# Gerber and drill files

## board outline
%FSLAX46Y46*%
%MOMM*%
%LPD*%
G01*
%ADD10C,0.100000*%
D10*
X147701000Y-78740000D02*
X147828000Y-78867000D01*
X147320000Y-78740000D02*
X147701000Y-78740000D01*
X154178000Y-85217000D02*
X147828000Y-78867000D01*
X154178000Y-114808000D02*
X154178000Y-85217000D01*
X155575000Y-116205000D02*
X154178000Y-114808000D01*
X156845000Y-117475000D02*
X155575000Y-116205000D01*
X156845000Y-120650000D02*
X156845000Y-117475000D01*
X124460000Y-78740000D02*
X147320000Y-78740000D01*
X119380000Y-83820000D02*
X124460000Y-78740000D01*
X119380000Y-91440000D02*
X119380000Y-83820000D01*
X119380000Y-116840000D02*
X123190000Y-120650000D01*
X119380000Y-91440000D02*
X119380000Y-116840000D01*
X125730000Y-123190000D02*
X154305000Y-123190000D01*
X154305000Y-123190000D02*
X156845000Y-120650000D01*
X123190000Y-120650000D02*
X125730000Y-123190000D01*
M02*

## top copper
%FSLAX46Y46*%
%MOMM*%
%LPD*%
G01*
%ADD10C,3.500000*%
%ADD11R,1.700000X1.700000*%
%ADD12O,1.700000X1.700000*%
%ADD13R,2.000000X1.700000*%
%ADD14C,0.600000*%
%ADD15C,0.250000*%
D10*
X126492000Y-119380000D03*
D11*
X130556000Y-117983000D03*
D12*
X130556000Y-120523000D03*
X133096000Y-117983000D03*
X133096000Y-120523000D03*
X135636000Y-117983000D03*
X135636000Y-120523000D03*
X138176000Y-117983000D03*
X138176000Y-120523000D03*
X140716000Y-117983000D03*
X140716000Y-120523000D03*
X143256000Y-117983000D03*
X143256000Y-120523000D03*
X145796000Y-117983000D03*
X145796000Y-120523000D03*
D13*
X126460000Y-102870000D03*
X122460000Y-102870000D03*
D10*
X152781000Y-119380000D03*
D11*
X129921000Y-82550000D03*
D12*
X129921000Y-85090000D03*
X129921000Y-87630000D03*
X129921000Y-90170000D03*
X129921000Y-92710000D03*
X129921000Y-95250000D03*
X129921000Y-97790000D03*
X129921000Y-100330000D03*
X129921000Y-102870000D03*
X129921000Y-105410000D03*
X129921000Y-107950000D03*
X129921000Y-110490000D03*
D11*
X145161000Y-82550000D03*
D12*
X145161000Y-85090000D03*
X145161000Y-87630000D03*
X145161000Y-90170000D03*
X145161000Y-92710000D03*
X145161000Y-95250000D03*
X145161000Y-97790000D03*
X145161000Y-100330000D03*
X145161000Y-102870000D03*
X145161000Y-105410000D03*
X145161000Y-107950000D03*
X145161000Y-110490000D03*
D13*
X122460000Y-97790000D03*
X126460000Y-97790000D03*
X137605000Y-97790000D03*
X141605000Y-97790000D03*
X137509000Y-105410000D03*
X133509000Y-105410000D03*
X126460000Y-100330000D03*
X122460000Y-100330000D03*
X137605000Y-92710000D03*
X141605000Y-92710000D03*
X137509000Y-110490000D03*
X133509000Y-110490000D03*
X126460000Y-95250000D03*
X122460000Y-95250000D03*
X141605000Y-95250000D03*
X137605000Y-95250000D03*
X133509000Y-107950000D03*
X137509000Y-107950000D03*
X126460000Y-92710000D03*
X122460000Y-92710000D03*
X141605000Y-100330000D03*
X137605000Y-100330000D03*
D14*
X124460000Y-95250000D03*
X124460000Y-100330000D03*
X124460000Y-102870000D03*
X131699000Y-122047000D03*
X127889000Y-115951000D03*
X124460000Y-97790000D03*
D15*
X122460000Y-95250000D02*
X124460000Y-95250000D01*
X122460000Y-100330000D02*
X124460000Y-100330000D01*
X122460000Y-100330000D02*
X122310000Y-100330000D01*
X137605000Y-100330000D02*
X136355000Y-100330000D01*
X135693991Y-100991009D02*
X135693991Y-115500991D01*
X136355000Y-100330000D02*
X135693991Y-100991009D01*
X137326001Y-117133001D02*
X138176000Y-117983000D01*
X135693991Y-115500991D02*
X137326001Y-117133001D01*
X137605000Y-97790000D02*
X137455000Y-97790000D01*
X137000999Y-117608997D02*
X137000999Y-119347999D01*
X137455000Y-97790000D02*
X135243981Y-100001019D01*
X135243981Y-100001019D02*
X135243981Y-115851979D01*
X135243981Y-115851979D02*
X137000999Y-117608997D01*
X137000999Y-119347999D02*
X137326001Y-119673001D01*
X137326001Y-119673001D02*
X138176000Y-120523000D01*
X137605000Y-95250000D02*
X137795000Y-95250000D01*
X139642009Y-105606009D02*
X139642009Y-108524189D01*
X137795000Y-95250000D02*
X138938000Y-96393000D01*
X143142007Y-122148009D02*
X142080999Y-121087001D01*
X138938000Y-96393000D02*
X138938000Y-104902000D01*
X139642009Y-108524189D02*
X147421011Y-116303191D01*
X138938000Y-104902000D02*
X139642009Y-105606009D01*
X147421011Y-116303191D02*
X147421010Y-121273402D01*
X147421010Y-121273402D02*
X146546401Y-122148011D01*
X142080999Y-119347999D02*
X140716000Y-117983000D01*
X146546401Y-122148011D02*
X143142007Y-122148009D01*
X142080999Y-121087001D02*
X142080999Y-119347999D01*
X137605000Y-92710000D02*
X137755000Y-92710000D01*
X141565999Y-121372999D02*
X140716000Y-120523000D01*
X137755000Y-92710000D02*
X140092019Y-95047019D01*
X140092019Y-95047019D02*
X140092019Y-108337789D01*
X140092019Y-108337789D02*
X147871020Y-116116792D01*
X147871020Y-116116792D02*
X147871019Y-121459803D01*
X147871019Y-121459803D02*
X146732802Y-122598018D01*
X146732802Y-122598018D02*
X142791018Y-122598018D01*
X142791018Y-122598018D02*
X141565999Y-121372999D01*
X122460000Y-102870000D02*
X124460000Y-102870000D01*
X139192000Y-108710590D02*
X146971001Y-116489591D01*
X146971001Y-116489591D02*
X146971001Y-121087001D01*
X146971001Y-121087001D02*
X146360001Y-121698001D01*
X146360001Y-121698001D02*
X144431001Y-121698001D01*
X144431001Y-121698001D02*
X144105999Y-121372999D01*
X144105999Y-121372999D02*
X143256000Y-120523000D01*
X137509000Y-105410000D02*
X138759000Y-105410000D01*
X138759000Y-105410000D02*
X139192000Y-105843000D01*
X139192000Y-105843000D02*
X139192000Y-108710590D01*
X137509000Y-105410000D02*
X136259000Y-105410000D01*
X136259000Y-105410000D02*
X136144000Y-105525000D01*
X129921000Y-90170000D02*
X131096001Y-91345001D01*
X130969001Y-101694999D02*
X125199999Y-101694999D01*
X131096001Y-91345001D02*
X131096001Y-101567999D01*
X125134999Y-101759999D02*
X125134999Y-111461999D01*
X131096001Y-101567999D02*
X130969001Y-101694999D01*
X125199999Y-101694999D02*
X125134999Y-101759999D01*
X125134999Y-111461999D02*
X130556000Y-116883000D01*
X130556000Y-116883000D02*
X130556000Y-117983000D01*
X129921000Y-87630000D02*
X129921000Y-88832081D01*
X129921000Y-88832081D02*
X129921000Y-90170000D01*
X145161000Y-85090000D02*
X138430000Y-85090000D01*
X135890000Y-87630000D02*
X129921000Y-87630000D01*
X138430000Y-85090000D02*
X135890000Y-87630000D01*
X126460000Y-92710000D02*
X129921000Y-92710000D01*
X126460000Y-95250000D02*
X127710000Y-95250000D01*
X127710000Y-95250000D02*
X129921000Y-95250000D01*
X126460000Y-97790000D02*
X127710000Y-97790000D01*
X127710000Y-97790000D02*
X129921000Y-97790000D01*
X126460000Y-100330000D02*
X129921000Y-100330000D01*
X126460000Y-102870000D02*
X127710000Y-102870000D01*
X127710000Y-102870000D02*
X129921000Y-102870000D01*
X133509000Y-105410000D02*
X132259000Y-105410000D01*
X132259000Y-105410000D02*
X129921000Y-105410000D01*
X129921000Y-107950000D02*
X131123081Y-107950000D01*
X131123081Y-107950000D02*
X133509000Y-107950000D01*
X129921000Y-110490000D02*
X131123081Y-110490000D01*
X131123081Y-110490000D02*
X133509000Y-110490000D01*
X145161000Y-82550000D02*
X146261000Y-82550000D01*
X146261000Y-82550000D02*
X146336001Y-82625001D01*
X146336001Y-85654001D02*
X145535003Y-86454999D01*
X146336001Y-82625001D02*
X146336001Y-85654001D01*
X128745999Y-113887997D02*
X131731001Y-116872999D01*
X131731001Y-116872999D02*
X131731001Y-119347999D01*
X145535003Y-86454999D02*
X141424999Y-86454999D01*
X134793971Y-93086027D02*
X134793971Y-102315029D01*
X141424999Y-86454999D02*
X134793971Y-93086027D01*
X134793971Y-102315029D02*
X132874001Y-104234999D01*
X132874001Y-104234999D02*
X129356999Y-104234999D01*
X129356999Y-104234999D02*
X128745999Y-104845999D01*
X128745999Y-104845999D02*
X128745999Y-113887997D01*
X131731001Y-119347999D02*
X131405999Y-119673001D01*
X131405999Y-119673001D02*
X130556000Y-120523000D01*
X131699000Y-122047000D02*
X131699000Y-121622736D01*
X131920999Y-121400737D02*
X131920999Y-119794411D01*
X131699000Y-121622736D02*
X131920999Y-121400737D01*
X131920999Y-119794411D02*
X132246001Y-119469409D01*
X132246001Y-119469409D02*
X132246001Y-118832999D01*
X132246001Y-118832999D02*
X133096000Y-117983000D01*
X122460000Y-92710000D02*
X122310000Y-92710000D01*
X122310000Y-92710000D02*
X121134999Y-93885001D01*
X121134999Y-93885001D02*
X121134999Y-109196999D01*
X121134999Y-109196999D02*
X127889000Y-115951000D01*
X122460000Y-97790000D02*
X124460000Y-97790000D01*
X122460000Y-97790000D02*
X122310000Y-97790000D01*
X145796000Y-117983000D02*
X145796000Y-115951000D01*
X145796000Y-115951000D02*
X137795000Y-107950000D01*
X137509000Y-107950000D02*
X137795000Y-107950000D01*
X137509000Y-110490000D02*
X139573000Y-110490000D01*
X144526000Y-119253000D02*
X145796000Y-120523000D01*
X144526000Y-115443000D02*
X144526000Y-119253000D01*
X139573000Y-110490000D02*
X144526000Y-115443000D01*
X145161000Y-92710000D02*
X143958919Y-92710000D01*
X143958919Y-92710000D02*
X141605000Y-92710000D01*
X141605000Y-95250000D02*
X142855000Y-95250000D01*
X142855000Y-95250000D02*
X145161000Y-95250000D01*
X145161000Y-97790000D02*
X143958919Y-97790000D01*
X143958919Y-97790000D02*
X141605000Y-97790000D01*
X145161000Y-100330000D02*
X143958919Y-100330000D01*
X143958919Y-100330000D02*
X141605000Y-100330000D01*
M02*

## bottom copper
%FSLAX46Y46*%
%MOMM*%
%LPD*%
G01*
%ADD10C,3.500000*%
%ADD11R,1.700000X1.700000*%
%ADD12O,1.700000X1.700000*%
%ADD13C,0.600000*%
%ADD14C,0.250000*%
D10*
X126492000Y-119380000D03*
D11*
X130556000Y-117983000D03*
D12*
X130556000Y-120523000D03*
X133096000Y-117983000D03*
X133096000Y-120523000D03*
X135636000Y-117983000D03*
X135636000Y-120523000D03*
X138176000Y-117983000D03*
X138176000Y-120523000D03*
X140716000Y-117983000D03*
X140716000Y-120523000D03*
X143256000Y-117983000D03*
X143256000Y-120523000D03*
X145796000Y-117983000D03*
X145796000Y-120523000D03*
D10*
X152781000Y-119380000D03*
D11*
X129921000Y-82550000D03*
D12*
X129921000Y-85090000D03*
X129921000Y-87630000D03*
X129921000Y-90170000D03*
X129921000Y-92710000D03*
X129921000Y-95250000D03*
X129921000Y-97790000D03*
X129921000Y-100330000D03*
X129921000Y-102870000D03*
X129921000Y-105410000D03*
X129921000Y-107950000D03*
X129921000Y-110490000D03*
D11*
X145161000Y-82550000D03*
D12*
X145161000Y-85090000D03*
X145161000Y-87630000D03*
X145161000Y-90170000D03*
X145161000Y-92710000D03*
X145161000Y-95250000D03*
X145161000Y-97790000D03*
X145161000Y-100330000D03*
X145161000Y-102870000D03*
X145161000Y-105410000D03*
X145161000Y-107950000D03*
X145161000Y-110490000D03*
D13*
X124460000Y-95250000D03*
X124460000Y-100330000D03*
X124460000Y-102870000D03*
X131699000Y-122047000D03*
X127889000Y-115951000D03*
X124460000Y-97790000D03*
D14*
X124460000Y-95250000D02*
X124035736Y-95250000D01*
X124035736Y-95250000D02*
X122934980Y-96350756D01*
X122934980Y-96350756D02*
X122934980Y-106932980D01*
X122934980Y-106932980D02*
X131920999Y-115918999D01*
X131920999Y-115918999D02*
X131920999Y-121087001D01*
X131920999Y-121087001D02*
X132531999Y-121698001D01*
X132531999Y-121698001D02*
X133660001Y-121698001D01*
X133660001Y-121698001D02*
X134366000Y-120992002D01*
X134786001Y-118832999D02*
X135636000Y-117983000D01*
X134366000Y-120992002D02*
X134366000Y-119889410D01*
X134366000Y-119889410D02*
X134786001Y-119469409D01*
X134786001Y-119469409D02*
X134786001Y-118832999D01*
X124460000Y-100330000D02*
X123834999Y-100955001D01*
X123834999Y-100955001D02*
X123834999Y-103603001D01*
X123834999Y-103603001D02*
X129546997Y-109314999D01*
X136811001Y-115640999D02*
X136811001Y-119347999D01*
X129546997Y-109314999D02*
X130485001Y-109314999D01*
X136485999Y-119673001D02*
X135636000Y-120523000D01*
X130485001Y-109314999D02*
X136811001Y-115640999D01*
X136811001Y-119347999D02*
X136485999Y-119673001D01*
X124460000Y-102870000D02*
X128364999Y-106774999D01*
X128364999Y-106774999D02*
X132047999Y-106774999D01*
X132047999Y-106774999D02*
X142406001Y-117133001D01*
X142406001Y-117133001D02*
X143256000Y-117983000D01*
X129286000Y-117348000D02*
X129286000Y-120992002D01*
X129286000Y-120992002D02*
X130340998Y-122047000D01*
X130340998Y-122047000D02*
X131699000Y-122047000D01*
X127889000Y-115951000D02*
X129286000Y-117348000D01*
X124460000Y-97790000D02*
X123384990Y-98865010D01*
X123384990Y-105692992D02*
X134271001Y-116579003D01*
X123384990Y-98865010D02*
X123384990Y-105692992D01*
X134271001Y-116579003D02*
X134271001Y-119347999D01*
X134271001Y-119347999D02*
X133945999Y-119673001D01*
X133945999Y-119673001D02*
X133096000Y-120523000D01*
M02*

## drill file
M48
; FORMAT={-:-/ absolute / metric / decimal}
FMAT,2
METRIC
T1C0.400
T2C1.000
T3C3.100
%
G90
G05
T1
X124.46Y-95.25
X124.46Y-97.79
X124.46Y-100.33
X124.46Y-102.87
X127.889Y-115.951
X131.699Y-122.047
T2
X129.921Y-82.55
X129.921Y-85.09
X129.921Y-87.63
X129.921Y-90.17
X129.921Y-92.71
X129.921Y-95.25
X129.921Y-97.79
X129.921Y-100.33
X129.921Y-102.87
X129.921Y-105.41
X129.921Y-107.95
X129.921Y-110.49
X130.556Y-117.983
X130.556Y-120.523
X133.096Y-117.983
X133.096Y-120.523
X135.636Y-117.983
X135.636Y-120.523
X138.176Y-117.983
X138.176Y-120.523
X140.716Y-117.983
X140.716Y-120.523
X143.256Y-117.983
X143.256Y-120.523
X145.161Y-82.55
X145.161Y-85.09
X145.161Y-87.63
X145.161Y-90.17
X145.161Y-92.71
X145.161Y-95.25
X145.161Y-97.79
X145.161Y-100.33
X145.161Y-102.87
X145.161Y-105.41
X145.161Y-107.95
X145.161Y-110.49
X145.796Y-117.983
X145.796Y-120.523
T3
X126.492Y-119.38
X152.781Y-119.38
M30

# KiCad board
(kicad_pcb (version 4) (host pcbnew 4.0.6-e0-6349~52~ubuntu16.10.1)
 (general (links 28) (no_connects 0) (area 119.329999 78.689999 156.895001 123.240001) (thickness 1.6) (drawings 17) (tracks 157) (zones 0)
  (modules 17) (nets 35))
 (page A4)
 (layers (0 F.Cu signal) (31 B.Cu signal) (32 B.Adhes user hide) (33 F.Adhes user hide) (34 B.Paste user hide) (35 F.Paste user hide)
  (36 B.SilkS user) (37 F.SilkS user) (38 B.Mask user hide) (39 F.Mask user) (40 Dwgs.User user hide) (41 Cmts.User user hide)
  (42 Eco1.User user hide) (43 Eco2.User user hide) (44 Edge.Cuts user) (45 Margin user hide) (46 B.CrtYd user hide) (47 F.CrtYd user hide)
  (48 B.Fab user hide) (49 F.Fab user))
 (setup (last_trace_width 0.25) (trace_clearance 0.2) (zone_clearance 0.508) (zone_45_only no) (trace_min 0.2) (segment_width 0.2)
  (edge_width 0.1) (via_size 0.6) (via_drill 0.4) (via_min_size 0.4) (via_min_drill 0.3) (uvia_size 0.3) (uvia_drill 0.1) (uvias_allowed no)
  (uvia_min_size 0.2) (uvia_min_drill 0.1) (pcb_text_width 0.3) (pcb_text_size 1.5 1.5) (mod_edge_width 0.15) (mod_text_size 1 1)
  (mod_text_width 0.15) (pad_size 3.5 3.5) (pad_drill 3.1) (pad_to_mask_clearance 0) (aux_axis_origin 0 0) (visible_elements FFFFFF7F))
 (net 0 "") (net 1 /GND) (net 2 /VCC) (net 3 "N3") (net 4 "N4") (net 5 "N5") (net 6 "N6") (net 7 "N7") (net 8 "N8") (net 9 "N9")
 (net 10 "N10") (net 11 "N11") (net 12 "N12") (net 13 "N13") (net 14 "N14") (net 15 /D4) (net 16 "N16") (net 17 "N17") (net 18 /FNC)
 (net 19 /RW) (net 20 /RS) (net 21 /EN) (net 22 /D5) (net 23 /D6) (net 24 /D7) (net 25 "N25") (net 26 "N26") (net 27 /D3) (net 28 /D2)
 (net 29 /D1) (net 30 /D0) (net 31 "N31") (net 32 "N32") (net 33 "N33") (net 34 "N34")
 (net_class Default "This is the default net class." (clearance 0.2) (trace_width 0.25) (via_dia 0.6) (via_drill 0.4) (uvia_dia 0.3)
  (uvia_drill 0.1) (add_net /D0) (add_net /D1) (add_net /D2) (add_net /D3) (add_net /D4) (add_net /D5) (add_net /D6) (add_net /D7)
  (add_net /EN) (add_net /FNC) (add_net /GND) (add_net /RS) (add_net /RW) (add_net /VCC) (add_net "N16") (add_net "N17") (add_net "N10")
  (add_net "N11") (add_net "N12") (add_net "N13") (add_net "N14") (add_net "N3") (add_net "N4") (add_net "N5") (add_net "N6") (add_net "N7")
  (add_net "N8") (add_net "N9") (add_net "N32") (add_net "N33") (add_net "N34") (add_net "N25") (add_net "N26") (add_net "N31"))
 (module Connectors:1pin (layer F.Cu) (at 126.492 119.38)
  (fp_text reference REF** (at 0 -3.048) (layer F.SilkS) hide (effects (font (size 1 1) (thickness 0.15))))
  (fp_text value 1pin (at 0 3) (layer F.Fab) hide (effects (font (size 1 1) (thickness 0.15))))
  (pad 1 thru_hole circle (at 0 0) (size 3.5 3.5) (drill 3.1) (layers *.Cu *.Mask)))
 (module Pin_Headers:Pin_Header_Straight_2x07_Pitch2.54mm (layer B.Cu) (at 130.556 117.983 270)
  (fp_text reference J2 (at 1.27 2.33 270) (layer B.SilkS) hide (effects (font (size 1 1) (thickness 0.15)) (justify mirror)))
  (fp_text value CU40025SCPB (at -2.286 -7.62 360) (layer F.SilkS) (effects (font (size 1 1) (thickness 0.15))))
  (pad 1 thru_hole rect (at 0 0 270) (size 1.7 1.7) (drill 1) (layers *.Cu *.Mask) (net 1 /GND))
  (pad 2 thru_hole oval (at 2.54 0 270) (size 1.7 1.7) (drill 1) (layers *.Cu *.Mask) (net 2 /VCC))
  (pad 3 thru_hole oval (at 0 -2.54 270) (size 1.7 1.7) (drill 1) (layers *.Cu *.Mask) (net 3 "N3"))
  (pad 4 thru_hole oval (at 2.54 -2.54 270) (size 1.7 1.7) (drill 1) (layers *.Cu *.Mask) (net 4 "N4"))
  (pad 5 thru_hole oval (at 0 -5.08 270) (size 1.7 1.7) (drill 1) (layers *.Cu *.Mask) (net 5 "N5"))
  (pad 6 thru_hole oval (at 2.54 -5.08 270) (size 1.7 1.7) (drill 1) (layers *.Cu *.Mask) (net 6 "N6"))
  (pad 7 thru_hole oval (at 0 -7.62 270) (size 1.7 1.7) (drill 1) (layers *.Cu *.Mask) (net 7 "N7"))
  (pad 8 thru_hole oval (at 2.54 -7.62 270) (size 1.7 1.7) (drill 1) (layers *.Cu *.Mask) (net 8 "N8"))
  (pad 9 thru_hole oval (at 0 -10.16 270) (size 1.7 1.7) (drill 1) (layers *.Cu *.Mask) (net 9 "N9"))
  (pad 10 thru_hole oval (at 2.54 -10.16 270) (size 1.7 1.7) (drill 1) (layers *.Cu *.Mask) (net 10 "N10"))
  (pad 11 thru_hole oval (at 0 -12.7 270) (size 1.7 1.7) (drill 1) (layers *.Cu *.Mask) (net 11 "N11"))
  (pad 12 thru_hole oval (at 2.54 -12.7 270) (size 1.7 1.7) (drill 1) (layers *.Cu *.Mask) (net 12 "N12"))
  (pad 13 thru_hole oval (at 0 -15.24 270) (size 1.7 1.7) (drill 1) (layers *.Cu *.Mask) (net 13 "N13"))
  (pad 14 thru_hole oval (at 2.54 -15.24 270) (size 1.7 1.7) (drill 1) (layers *.Cu *.Mask) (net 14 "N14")))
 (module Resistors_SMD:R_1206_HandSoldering (layer F.Cu) (at 124.46 102.87 180)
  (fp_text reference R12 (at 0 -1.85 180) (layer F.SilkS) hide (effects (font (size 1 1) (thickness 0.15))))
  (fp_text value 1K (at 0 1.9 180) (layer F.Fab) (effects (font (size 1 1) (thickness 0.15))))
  (pad 1 smd rect (at -2 0 180) (size 2 1.7) (layers F.Cu F.Paste F.Mask) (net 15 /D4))
  (pad 2 smd rect (at 2 0 180) (size 2 1.7) (layers F.Cu F.Paste F.Mask) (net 11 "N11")))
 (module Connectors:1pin (layer F.Cu) (at 152.781 119.38)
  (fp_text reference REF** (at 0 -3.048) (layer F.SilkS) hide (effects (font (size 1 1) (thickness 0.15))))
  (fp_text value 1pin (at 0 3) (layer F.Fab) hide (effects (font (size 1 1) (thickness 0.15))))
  (pad 1 thru_hole circle (at 0 0) (size 3.5 3.5) (drill 3.1) (layers *.Cu *.Mask)))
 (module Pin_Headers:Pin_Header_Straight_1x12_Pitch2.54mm (layer F.Cu) (at 129.921 82.55)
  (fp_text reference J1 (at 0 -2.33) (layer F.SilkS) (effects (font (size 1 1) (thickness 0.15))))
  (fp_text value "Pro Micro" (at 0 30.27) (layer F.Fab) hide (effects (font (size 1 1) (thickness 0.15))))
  (pad 1 thru_hole rect (at 0 0) (size 1.7 1.7) (drill 1) (layers *.Cu *.Mask) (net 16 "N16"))
  (pad 2 thru_hole oval (at 0 2.54) (size 1.7 1.7) (drill 1) (layers *.Cu *.Mask) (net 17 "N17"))
  (pad 3 thru_hole oval (at 0 5.08) (size 1.7 1.7) (drill 1) (layers *.Cu *.Mask) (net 1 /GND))
  (pad 4 thru_hole oval (at 0 7.62) (size 1.7 1.7) (drill 1) (layers *.Cu *.Mask) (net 1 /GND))
  (pad 5 thru_hole oval (at 0 10.16) (size 1.7 1.7) (drill 1) (layers *.Cu *.Mask) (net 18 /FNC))
  (pad 6 thru_hole oval (at 0 12.7) (size 1.7 1.7) (drill 1) (layers *.Cu *.Mask) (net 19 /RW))
  (pad 7 thru_hole oval (at 0 15.24) (size 1.7 1.7) (drill 1) (layers *.Cu *.Mask) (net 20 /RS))
  (pad 8 thru_hole oval (at 0 17.78) (size 1.7 1.7) (drill 1) (layers *.Cu *.Mask) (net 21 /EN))
  (pad 9 thru_hole oval (at 0 20.32) (size 1.7 1.7) (drill 1) (layers *.Cu *.Mask) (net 15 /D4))
  (pad 10 thru_hole oval (at 0 22.86) (size 1.7 1.7) (drill 1) (layers *.Cu *.Mask) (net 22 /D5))
  (pad 11 thru_hole oval (at 0 25.4) (size 1.7 1.7) (drill 1) (layers *.Cu *.Mask) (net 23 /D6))
  (pad 12 thru_hole oval (at 0 27.94) (size 1.7 1.7) (drill 1) (layers *.Cu *.Mask) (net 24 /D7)))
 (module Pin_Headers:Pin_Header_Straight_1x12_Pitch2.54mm (layer F.Cu) (at 145.161 82.55)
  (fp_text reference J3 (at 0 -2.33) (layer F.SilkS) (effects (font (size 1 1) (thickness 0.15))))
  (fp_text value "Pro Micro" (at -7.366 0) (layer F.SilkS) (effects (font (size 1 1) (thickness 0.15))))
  (pad 1 thru_hole rect (at 0 0) (size 1.7 1.7) (drill 1) (layers *.Cu *.Mask) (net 2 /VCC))
  (pad 2 thru_hole oval (at 0 2.54) (size 1.7 1.7) (drill 1) (layers *.Cu *.Mask) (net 1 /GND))
  (pad 3 thru_hole oval (at 0 5.08) (size 1.7 1.7) (drill 1) (layers *.Cu *.Mask) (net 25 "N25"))
  (pad 4 thru_hole oval (at 0 7.62) (size 1.7 1.7) (drill 1) (layers *.Cu *.Mask) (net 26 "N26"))
  (pad 5 thru_hole oval (at 0 10.16) (size 1.7 1.7) (drill 1) (layers *.Cu *.Mask) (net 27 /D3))
  (pad 6 thru_hole oval (at 0 12.7) (size 1.7 1.7) (drill 1) (layers *.Cu *.Mask) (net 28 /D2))
  (pad 7 thru_hole oval (at 0 15.24) (size 1.7 1.7) (drill 1) (layers *.Cu *.Mask) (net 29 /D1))
  (pad 8 thru_hole oval (at 0 17.78) (size 1.7 1.7) (drill 1) (layers *.Cu *.Mask) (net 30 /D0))
  (pad 9 thru_hole oval (at 0 20.32) (size 1.7 1.7) (drill 1) (layers *.Cu *.Mask) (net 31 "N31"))
  (pad 10 thru_hole oval (at 0 22.86) (size 1.7 1.7) (drill 1) (layers *.Cu *.Mask) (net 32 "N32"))
  (pad 11 thru_hole oval (at 0 25.4) (size 1.7 1.7) (drill 1) (layers *.Cu *.Mask) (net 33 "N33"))
  (pad 12 thru_hole oval (at 0 27.94) (size 1.7 1.7) (drill 1) (layers *.Cu *.Mask) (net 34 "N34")))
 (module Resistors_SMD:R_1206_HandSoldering (layer F.Cu) (at 124.46 97.79)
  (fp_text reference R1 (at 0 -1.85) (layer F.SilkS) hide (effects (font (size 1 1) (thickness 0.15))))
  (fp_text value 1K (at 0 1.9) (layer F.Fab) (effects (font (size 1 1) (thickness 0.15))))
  (pad 1 smd rect (at -2 0) (size 2 1.7) (layers F.Cu F.Paste F.Mask) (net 4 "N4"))
  (pad 2 smd rect (at 2 0) (size 2 1.7) (layers F.Cu F.Paste F.Mask) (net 20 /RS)))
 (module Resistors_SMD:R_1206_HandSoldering (layer F.Cu) (at 139.605 97.79)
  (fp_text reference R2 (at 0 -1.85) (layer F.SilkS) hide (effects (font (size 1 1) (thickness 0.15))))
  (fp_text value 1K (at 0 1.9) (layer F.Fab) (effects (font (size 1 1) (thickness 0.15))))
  (pad 1 smd rect (at -2 0) (size 2 1.7) (layers F.Cu F.Paste F.Mask) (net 8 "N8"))
  (pad 2 smd rect (at 2 0) (size 2 1.7) (layers F.Cu F.Paste F.Mask) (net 29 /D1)))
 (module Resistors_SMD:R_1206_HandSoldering (layer F.Cu) (at 135.509 105.41 180)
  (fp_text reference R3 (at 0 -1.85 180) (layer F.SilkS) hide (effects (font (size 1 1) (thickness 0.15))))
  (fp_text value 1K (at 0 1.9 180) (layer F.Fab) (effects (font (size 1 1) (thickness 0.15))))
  (pad 1 smd rect (at -2 0 180) (size 2 1.7) (layers F.Cu F.Paste F.Mask) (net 12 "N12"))
  (pad 2 smd rect (at 2 0 180) (size 2 1.7) (layers F.Cu F.Paste F.Mask) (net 22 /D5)))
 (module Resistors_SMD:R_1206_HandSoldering (layer F.Cu) (at 124.46 100.33 180)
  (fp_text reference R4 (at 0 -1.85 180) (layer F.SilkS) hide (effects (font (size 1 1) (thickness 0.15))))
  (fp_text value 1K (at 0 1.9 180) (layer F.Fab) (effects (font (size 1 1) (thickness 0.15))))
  (pad 1 smd rect (at -2 0 180) (size 2 1.7) (layers F.Cu F.Paste F.Mask) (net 21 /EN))
  (pad 2 smd rect (at 2 0 180) (size 2 1.7) (layers F.Cu F.Paste F.Mask) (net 6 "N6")))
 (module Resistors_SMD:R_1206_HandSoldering (layer F.Cu) (at 139.605 92.71)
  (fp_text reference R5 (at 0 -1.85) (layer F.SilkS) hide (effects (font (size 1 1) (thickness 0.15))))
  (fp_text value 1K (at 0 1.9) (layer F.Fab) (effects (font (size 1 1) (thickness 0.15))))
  (pad 1 smd rect (at -2 0) (size 2 1.7) (layers F.Cu F.Paste F.Mask) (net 10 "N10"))
  (pad 2 smd rect (at 2 0) (size 2 1.7) (layers F.Cu F.Paste F.Mask) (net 27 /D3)))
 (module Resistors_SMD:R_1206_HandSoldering (layer F.Cu) (at 135.509 110.49 180)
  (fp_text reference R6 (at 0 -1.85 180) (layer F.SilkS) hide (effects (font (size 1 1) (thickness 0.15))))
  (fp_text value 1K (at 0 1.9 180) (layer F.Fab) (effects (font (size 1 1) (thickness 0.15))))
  (pad 1 smd rect (at -2 0 180) (size 2 1.7) (layers F.Cu F.Paste F.Mask) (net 14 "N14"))
  (pad 2 smd rect (at 2 0 180) (size 2 1.7) (layers F.Cu F.Paste F.Mask) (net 24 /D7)))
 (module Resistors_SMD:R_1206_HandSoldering (layer F.Cu) (at 124.46 95.25 180)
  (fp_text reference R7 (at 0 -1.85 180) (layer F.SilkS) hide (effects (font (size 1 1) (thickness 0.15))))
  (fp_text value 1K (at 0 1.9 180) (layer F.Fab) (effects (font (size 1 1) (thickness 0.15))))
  (pad 1 smd rect (at -2 0 180) (size 2 1.7) (layers F.Cu F.Paste F.Mask) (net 19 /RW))
  (pad 2 smd rect (at 2 0 180) (size 2 1.7) (layers F.Cu F.Paste F.Mask) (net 5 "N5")))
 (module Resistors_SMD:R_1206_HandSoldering (layer F.Cu) (at 139.605 95.25 180)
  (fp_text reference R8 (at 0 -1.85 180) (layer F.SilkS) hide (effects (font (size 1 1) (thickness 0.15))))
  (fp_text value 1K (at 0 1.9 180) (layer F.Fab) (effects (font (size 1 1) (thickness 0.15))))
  (pad 1 smd rect (at -2 0 180) (size 2 1.7) (layers F.Cu F.Paste F.Mask) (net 28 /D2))
  (pad 2 smd rect (at 2 0 180) (size 2 1.7) (layers F.Cu F.Paste F.Mask) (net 9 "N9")))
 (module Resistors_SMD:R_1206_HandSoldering (layer F.Cu) (at 135.509 107.95)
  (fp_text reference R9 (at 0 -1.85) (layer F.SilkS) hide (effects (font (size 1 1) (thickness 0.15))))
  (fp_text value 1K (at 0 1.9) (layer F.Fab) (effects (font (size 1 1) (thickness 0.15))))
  (pad 1 smd rect (at -2 0) (size 2 1.7) (layers F.Cu F.Paste F.Mask) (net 23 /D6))
  (pad 2 smd rect (at 2 0) (size 2 1.7) (layers F.Cu F.Paste F.Mask) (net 13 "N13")))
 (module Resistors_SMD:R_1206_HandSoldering (layer F.Cu) (at 124.46 92.71 180)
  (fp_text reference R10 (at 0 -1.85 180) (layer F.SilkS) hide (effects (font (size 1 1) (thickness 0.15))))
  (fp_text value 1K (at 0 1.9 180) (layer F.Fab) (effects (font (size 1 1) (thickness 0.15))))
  (pad 1 smd rect (at -2 0 180) (size 2 1.7) (layers F.Cu F.Paste F.Mask) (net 18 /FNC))
  (pad 2 smd rect (at 2 0 180) (size 2 1.7) (layers F.Cu F.Paste F.Mask) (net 3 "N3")))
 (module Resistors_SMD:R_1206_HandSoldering (layer F.Cu) (at 139.605 100.33 180)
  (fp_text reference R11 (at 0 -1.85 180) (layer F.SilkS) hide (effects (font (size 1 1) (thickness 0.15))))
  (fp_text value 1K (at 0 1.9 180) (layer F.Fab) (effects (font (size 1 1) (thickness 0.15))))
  (pad 1 smd rect (at -2 0 180) (size 2 1.7) (layers F.Cu F.Paste F.Mask) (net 30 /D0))
  (pad 2 smd rect (at 2 0 180) (size 2 1.7) (layers F.Cu F.Paste F.Mask) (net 7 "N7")))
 (gr_line (start 147.701 78.74) (end 147.828 78.867) (layer Edge.Cuts) (width 0.1))
 (gr_line (start 147.32 78.74) (end 147.701 78.74) (layer Edge.Cuts) (width 0.1))
 (gr_line (start 154.178 85.217) (end 147.828 78.867) (layer Edge.Cuts) (width 0.1))
 (gr_line (start 154.178 114.808) (end 154.178 85.217) (layer Edge.Cuts) (width 0.1))
 (gr_line (start 155.575 116.205) (end 154.178 114.808) (layer Edge.Cuts) (width 0.1))
 (gr_line (start 156.845 117.475) (end 155.575 116.205) (layer Edge.Cuts) (width 0.1))
 (gr_line (start 156.845 120.65) (end 156.845 117.475) (layer Edge.Cuts) (width 0.1))
 (gr_line (start 124.46 78.74) (end 147.32 78.74) (layer Edge.Cuts) (width 0.1))
 (gr_line (start 119.38 83.82) (end 124.46 78.74) (layer Edge.Cuts) (width 0.1))
 (gr_line (start 119.38 91.44) (end 119.38 83.82) (layer Edge.Cuts) (width 0.1))
 (gr_line (start 119.38 116.84) (end 123.19 120.65) (layer Edge.Cuts) (width 0.1))
 (gr_line (start 119.38 91.44) (end 119.38 116.84) (layer Edge.Cuts) (width 0.1))
 (gr_line (start 125.73 123.19) (end 154.305 123.19) (angle 90) (layer Edge.Cuts) (width 0.1))
 (gr_line (start 154.305 123.19) (end 156.845 120.65) (angle 90) (layer Edge.Cuts) (width 0.1))
 (gr_line (start 123.19 120.65) (end 125.73 123.19) (angle 90) (layer Edge.Cuts) (width 0.1))
 (segment (start 124.46 95.25) (end 124.035736 95.25) (width 0.25) (layer B.Cu) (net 5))
 (segment (start 124.035736 95.25) (end 122.93498 96.350756) (width 0.25) (layer B.Cu) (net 5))
 (segment (start 122.93498 96.350756) (end 122.93498 106.93298) (width 0.25) (layer B.Cu) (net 5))
 (segment (start 122.93498 106.93298) (end 131.920999 115.918999) (width 0.25) (layer B.Cu) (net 5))
 (segment (start 131.920999 115.918999) (end 131.920999 121.087001) (width 0.25) (layer B.Cu) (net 5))
 (segment (start 131.920999 121.087001) (end 132.531999 121.698001) (width 0.25) (layer B.Cu) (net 5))
 (segment (start 132.531999 121.698001) (end 133.660001 121.698001) (width 0.25) (layer B.Cu) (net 5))
 (segment (start 133.660001 121.698001) (end 134.366 120.992002) (width 0.25) (layer B.Cu) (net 5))
 (segment (start 134.786001 118.832999) (end 135.636 117.983) (width 0.25) (layer B.Cu) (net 5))
 (segment (start 134.366 120.992002) (end 134.366 119.88941) (width 0.25) (layer B.Cu) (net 5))
 (segment (start 134.366 119.88941) (end 134.786001 119.469409) (width 0.25) (layer B.Cu) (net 5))
 (segment (start 134.786001 119.469409) (end 134.786001 118.832999) (width 0.25) (layer B.Cu) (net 5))
 (segment (start 122.46 95.25) (end 124.46 95.25) (width 0.25) (layer F.Cu) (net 5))
 (via (at 124.46 95.25) (size 0.6) (drill 0.4) (layers F.Cu B.Cu) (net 5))
 (segment (start 124.46 100.33) (end 123.834999 100.955001) (width 0.25) (layer B.Cu) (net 6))
 (segment (start 123.834999 100.955001) (end 123.834999 103.603001) (width 0.25) (layer B.Cu) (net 6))
 (segment (start 123.834999 103.603001) (end 129.546997 109.314999) (width 0.25) (layer B.Cu) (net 6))
 (segment (start 136.811001 115.640999) (end 136.811001 119.347999) (width 0.25) (layer B.Cu) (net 6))
 (segment (start 129.546997 109.314999) (end 130.485001 109.314999) (width 0.25) (layer B.Cu) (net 6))
 (segment (start 136.485999 119.673001) (end 135.636 120.523) (width 0.25) (layer B.Cu) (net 6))
 (segment (start 130.485001 109.314999) (end 136.811001 115.640999) (width 0.25) (layer B.Cu) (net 6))
 (segment (start 136.811001 119.347999) (end 136.485999 119.673001) (width 0.25) (layer B.Cu) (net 6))
 (segment (start 122.46 100.33) (end 124.46 100.33) (width 0.25) (layer F.Cu) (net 6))
 (via (at 124.46 100.33) (size 0.6) (drill 0.4) (layers F.Cu B.Cu) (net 6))
 (segment (start 122.46 100.33) (end 122.31 100.33) (width 0.25) (layer F.Cu) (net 6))
 (segment (start 137.605 100.33) (end 136.355 100.33) (width 0.25) (layer F.Cu) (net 7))
 (segment (start 135.693991 100.991009) (end 135.693991 115.500991) (width 0.25) (layer F.Cu) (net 7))
 (segment (start 136.355 100.33) (end 135.693991 100.991009) (width 0.25) (layer F.Cu) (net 7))
 (segment (start 137.326001 117.133001) (end 138.176 117.983) (width 0.25) (layer F.Cu) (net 7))
 (segment (start 135.693991 115.500991) (end 137.326001 117.133001) (width 0.25) (layer F.Cu) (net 7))
 (segment (start 137.605 97.79) (end 137.455 97.79) (width 0.25) (layer F.Cu) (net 8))
 (segment (start 137.000999 117.608997) (end 137.000999 119.347999) (width 0.25) (layer F.Cu) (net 8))
 (segment (start 137.455 97.79) (end 135.243981 100.001019) (width 0.25) (layer F.Cu) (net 8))
 (segment (start 135.243981 100.001019) (end 135.243981 115.851979) (width 0.25) (layer F.Cu) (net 8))
 (segment (start 135.243981 115.851979) (end 137.000999 117.608997) (width 0.25) (layer F.Cu) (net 8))
 (segment (start 137.000999 119.347999) (end 137.326001 119.673001) (width 0.25) (layer F.Cu) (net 8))
 (segment (start 137.326001 119.673001) (end 138.176 120.523) (width 0.25) (layer F.Cu) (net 8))
 (segment (start 137.605 95.25) (end 137.795 95.25) (width 0.25) (layer F.Cu) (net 9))
 (segment (start 139.642009 105.606009) (end 139.642009 108.524189) (width 0.25) (layer F.Cu) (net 9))
 (segment (start 137.795 95.25) (end 138.938 96.393) (width 0.25) (layer F.Cu) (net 9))
 (segment (start 143.142007 122.148009) (end 142.080999 121.087001) (width 0.25) (layer F.Cu) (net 9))
 (segment (start 138.938 96.393) (end 138.938 104.902) (width 0.25) (layer F.Cu) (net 9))
 (segment (start 139.642009 108.524189) (end 147.421011 116.303191) (width 0.25) (layer F.Cu) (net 9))
 (segment (start 138.938 104.902) (end 139.642009 105.606009) (width 0.25) (layer F.Cu) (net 9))
 (segment (start 147.421011 116.303191) (end 147.42101 121.273402) (width 0.25) (layer F.Cu) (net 9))
 (segment (start 147.42101 121.273402) (end 146.546401 122.148011) (width 0.25) (layer F.Cu) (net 9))
 (segment (start 142.080999 119.347999) (end 140.716 117.983) (width 0.25) (layer F.Cu) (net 9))
 (segment (start 146.546401 122.148011) (end 143.142007 122.148009) (width 0.25) (layer F.Cu) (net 9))
 (segment (start 142.080999 121.087001) (end 142.080999 119.347999) (width 0.25) (layer F.Cu) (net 9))
 (segment (start 137.605 92.71) (end 137.755 92.71) (width 0.25) (layer F.Cu) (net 10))
 (segment (start 141.565999 121.372999) (end 140.716 120.523) (width 0.25) (layer F.Cu) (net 10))
 (segment (start 137.755 92.71) (end 140.092019 95.047019) (width 0.25) (layer F.Cu) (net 10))
 (segment (start 140.092019 95.047019) (end 140.092019 108.337789) (width 0.25) (layer F.Cu) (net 10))
 (segment (start 140.092019 108.337789) (end 147.87102 116.116792) (width 0.25) (layer F.Cu) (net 10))
 (segment (start 147.87102 116.116792) (end 147.871019 121.459803) (width 0.25) (layer F.Cu) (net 10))
 (segment (start 147.871019 121.459803) (end 146.732802 122.598018) (width 0.25) (layer F.Cu) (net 10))
 (segment (start 146.732802 122.598018) (end 142.791018 122.598018) (width 0.25) (layer F.Cu) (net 10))
 (segment (start 142.791018 122.598018) (end 141.565999 121.372999) (width 0.25) (layer F.Cu) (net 10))
 (segment (start 124.46 102.87) (end 128.364999 106.774999) (width 0.25) (layer B.Cu) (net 11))
 (segment (start 128.364999 106.774999) (end 132.047999 106.774999) (width 0.25) (layer B.Cu) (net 11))
 (segment (start 132.047999 106.774999) (end 142.406001 117.133001) (width 0.25) (layer B.Cu) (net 11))
 (segment (start 142.406001 117.133001) (end 143.256 117.983) (width 0.25) (layer B.Cu) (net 11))
 (segment (start 122.46 102.87) (end 124.46 102.87) (width 0.25) (layer F.Cu) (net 11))
 (via (at 124.46 102.87) (size 0.6) (drill 0.4) (layers F.Cu B.Cu) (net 11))
 (segment (start 139.192 108.71059) (end 146.971001 116.489591) (width 0.25) (layer F.Cu) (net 12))
 (segment (start 146.971001 116.489591) (end 146.971001 121.087001) (width 0.25) (layer F.Cu) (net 12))
 (segment (start 146.971001 121.087001) (end 146.360001 121.698001) (width 0.25) (layer F.Cu) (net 12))
 (segment (start 146.360001 121.698001) (end 144.431001 121.698001) (width 0.25) (layer F.Cu) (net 12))
 (segment (start 144.431001 121.698001) (end 144.105999 121.372999) (width 0.25) (layer F.Cu) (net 12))
 (segment (start 144.105999 121.372999) (end 143.256 120.523) (width 0.25) (layer F.Cu) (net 12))
 (segment (start 137.509 105.41) (end 138.759 105.41) (width 0.25) (layer F.Cu) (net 12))
 (segment (start 138.759 105.41) (end 139.192 105.843) (width 0.25) (layer F.Cu) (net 12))
 (segment (start 139.192 105.843) (end 139.192 108.71059) (width 0.25) (layer F.Cu) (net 12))
 (segment (start 137.509 105.41) (end 136.259 105.41) (width 0.25) (layer F.Cu) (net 12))
 (segment (start 136.259 105.41) (end 136.144 105.525) (width 0.25) (layer F.Cu) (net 12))
 (segment (start 129.921 90.17) (end 131.096001 91.345001) (width 0.25) (layer F.Cu) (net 1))
 (segment (start 130.969001 101.694999) (end 125.199999 101.694999) (width 0.25) (layer F.Cu) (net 1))
 (segment (start 131.096001 91.345001) (end 131.096001 101.567999) (width 0.25) (layer F.Cu) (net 1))
 (segment (start 125.134999 101.759999) (end 125.134999 111.461999) (width 0.25) (layer F.Cu) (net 1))
 (segment (start 131.096001 101.567999) (end 130.969001 101.694999) (width 0.25) (layer F.Cu) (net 1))
 (segment (start 125.199999 101.694999) (end 125.134999 101.759999) (width 0.25) (layer F.Cu) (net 1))
 (segment (start 125.134999 111.461999) (end 130.556 116.883) (width 0.25) (layer F.Cu) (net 1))
 (segment (start 130.556 116.883) (end 130.556 117.983) (width 0.25) (layer F.Cu) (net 1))
 (segment (start 129.921 87.63) (end 129.921 88.832081) (width 0.25) (layer F.Cu) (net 1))
 (segment (start 129.921 88.832081) (end 129.921 90.17) (width 0.25) (layer F.Cu) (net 1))
 (segment (start 145.161 85.09) (end 138.43 85.09) (width 0.25) (layer F.Cu) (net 1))
 (segment (start 135.89 87.63) (end 129.921 87.63) (width 0.25) (layer F.Cu) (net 1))
 (segment (start 138.43 85.09) (end 135.89 87.63) (width 0.25) (layer F.Cu) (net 1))
 (segment (start 126.46 92.71) (end 129.921 92.71) (width 0.25) (layer F.Cu) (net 18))
 (segment (start 126.46 95.25) (end 127.71 95.25) (width 0.25) (layer F.Cu) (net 19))
 (segment (start 127.71 95.25) (end 129.921 95.25) (width 0.25) (layer F.Cu) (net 19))
 (segment (start 126.46 97.79) (end 127.71 97.79) (width 0.25) (layer F.Cu) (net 20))
 (segment (start 127.71 97.79) (end 129.921 97.79) (width 0.25) (layer F.Cu) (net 20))
 (segment (start 126.46 100.33) (end 129.921 100.33) (width 0.25) (layer F.Cu) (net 21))
 (segment (start 126.46 102.87) (end 127.71 102.87) (width 0.25) (layer F.Cu) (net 15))
 (segment (start 127.71 102.87) (end 129.921 102.87) (width 0.25) (layer F.Cu) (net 15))
 (segment (start 133.509 105.41) (end 132.259 105.41) (width 0.25) (layer F.Cu) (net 22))
 (segment (start 132.259 105.41) (end 129.921 105.41) (width 0.25) (layer F.Cu) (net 22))
 (segment (start 129.921 107.95) (end 131.123081 107.95) (width 0.25) (layer F.Cu) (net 23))
 (segment (start 131.123081 107.95) (end 133.509 107.95) (width 0.25) (layer F.Cu) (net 23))
 (segment (start 129.921 110.49) (end 131.123081 110.49) (width 0.25) (layer F.Cu) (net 24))
 (segment (start 131.123081 110.49) (end 133.509 110.49) (width 0.25) (layer F.Cu) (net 24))
 (segment (start 145.161 82.55) (end 146.261 82.55) (width 0.25) (layer F.Cu) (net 2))
 (segment (start 146.261 82.55) (end 146.336001 82.625001) (width 0.25) (layer F.Cu) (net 2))
 (segment (start 146.336001 85.654001) (end 145.535003 86.454999) (width 0.25) (layer F.Cu) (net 2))
 (segment (start 146.336001 82.625001) (end 146.336001 85.654001) (width 0.25) (layer F.Cu) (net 2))
 (segment (start 128.745999 113.887997) (end 131.731001 116.872999) (width 0.25) (layer F.Cu) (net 2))
 (segment (start 131.731001 116.872999) (end 131.731001 119.347999) (width 0.25) (layer F.Cu) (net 2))
 (segment (start 145.535003 86.454999) (end 141.424999 86.454999) (width 0.25) (layer F.Cu) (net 2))
 (segment (start 134.793971 93.086027) (end 134.793971 102.315029) (width 0.25) (layer F.Cu) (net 2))
 (segment (start 141.424999 86.454999) (end 134.793971 93.086027) (width 0.25) (layer F.Cu) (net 2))
 (segment (start 134.793971 102.315029) (end 132.874001 104.234999) (width 0.25) (layer F.Cu) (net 2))
 (segment (start 132.874001 104.234999) (end 129.356999 104.234999) (width 0.25) (layer F.Cu) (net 2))
 (segment (start 129.356999 104.234999) (end 128.745999 104.845999) (width 0.25) (layer F.Cu) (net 2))
 (segment (start 128.745999 104.845999) (end 128.745999 113.887997) (width 0.25) (layer F.Cu) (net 2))
 (segment (start 131.731001 119.347999) (end 131.405999 119.673001) (width 0.25) (layer F.Cu) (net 2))
 (segment (start 131.405999 119.673001) (end 130.556 120.523) (width 0.25) (layer F.Cu) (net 2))
 (segment (start 131.699 122.047) (end 131.699 121.622736) (width 0.25) (layer F.Cu) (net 3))
 (segment (start 131.920999 121.400737) (end 131.920999 119.794411) (width 0.25) (layer F.Cu) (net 3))
 (segment (start 131.699 121.622736) (end 131.920999 121.400737) (width 0.25) (layer F.Cu) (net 3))
 (segment (start 131.920999 119.794411) (end 132.246001 119.469409) (width 0.25) (layer F.Cu) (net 3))
 (segment (start 132.246001 119.469409) (end 132.246001 118.832999) (width 0.25) (layer F.Cu) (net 3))
 (segment (start 132.246001 118.832999) (end 133.096 117.983) (width 0.25) (layer F.Cu) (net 3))
 (segment (start 129.286 117.348) (end 129.286 120.992002) (width 0.25) (layer B.Cu) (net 3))
 (segment (start 129.286 120.992002) (end 130.340998 122.047) (width 0.25) (layer B.Cu) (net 3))
 (segment (start 130.340998 122.047) (end 131.699 122.047) (width 0.25) (layer B.Cu) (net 3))
 (via (at 131.699 122.047) (size 0.6) (drill 0.4) (layers F.Cu B.Cu) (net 3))
 (segment (start 127.889 115.951) (end 129.286 117.348) (width 0.25) (layer B.Cu) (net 3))
 (segment (start 122.46 92.71) (end 122.31 92.71) (width 0.25) (layer F.Cu) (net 3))
 (segment (start 122.31 92.71) (end 121.134999 93.885001) (width 0.25) (layer F.Cu) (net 3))
 (segment (start 121.134999 93.885001) (end 121.134999 109.196999) (width 0.25) (layer F.Cu) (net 3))
 (segment (start 121.134999 109.196999) (end 127.889 115.951) (width 0.25) (layer F.Cu) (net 3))
 (via (at 127.889 115.951) (size 0.6) (drill 0.4) (layers F.Cu B.Cu) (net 3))
 (segment (start 124.46 97.79) (end 123.38499 98.86501) (width 0.25) (layer B.Cu) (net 4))
 (segment (start 123.38499 105.692992) (end 134.271001 116.579003) (width 0.25) (layer B.Cu) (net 4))
 (segment (start 123.38499 98.86501) (end 123.38499 105.692992) (width 0.25) (layer B.Cu) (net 4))
 (segment (start 134.271001 116.579003) (end 134.271001 119.347999) (width 0.25) (layer B.Cu) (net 4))
 (segment (start 134.271001 119.347999) (end 133.945999 119.673001) (width 0.25) (layer B.Cu) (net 4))
 (segment (start 133.945999 119.673001) (end 133.096 120.523) (width 0.25) (layer B.Cu) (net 4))
 (segment (start 122.46 97.79) (end 124.46 97.79) (width 0.25) (layer F.Cu) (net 4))
 (via (at 124.46 97.79) (size 0.6) (drill 0.4) (layers F.Cu B.Cu) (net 4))
 (segment (start 122.46 97.79) (end 122.31 97.79) (width 0.25) (layer F.Cu) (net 4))
 (segment (start 145.796 117.983) (end 145.796 115.951) (width 0.25) (layer F.Cu) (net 13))
 (segment (start 145.796 115.951) (end 137.795 107.95) (width 0.25) (layer F.Cu) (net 13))
 (segment (start 137.509 107.95) (end 137.795 107.95) (width 0.25) (layer F.Cu) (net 13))
 (segment (start 137.509 110.49) (end 139.573 110.49) (width 0.25) (layer F.Cu) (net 14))
 (segment (start 144.526 119.253) (end 145.796 120.523) (width 0.25) (layer F.Cu) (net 14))
 (segment (start 144.526 115.443) (end 144.526 119.253) (width 0.25) (layer F.Cu) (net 14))
 (segment (start 139.573 110.49) (end 144.526 115.443) (width 0.25) (layer F.Cu) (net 14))
 (segment (start 145.161 92.71) (end 143.958919 92.71) (width 0.25) (layer F.Cu) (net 27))
 (segment (start 143.958919 92.71) (end 141.605 92.71) (width 0.25) (layer F.Cu) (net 27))
 (segment (start 141.605 95.25) (end 142.855 95.25) (width 0.25) (layer F.Cu) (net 28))
 (segment (start 142.855 95.25) (end 145.161 95.25) (width 0.25) (layer F.Cu) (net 28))
 (segment (start 145.161 97.79) (end 143.958919 97.79) (width 0.25) (layer F.Cu) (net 29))
 (segment (start 143.958919 97.79) (end 141.605 97.79) (width 0.25) (layer F.Cu) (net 29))
 (segment (start 145.161 100.33) (end 143.958919 100.33) (width 0.25) (layer F.Cu) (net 30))
 (segment (start 143.958919 100.33) (end 141.605 100.33) (width 0.25) (layer F.Cu) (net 30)))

